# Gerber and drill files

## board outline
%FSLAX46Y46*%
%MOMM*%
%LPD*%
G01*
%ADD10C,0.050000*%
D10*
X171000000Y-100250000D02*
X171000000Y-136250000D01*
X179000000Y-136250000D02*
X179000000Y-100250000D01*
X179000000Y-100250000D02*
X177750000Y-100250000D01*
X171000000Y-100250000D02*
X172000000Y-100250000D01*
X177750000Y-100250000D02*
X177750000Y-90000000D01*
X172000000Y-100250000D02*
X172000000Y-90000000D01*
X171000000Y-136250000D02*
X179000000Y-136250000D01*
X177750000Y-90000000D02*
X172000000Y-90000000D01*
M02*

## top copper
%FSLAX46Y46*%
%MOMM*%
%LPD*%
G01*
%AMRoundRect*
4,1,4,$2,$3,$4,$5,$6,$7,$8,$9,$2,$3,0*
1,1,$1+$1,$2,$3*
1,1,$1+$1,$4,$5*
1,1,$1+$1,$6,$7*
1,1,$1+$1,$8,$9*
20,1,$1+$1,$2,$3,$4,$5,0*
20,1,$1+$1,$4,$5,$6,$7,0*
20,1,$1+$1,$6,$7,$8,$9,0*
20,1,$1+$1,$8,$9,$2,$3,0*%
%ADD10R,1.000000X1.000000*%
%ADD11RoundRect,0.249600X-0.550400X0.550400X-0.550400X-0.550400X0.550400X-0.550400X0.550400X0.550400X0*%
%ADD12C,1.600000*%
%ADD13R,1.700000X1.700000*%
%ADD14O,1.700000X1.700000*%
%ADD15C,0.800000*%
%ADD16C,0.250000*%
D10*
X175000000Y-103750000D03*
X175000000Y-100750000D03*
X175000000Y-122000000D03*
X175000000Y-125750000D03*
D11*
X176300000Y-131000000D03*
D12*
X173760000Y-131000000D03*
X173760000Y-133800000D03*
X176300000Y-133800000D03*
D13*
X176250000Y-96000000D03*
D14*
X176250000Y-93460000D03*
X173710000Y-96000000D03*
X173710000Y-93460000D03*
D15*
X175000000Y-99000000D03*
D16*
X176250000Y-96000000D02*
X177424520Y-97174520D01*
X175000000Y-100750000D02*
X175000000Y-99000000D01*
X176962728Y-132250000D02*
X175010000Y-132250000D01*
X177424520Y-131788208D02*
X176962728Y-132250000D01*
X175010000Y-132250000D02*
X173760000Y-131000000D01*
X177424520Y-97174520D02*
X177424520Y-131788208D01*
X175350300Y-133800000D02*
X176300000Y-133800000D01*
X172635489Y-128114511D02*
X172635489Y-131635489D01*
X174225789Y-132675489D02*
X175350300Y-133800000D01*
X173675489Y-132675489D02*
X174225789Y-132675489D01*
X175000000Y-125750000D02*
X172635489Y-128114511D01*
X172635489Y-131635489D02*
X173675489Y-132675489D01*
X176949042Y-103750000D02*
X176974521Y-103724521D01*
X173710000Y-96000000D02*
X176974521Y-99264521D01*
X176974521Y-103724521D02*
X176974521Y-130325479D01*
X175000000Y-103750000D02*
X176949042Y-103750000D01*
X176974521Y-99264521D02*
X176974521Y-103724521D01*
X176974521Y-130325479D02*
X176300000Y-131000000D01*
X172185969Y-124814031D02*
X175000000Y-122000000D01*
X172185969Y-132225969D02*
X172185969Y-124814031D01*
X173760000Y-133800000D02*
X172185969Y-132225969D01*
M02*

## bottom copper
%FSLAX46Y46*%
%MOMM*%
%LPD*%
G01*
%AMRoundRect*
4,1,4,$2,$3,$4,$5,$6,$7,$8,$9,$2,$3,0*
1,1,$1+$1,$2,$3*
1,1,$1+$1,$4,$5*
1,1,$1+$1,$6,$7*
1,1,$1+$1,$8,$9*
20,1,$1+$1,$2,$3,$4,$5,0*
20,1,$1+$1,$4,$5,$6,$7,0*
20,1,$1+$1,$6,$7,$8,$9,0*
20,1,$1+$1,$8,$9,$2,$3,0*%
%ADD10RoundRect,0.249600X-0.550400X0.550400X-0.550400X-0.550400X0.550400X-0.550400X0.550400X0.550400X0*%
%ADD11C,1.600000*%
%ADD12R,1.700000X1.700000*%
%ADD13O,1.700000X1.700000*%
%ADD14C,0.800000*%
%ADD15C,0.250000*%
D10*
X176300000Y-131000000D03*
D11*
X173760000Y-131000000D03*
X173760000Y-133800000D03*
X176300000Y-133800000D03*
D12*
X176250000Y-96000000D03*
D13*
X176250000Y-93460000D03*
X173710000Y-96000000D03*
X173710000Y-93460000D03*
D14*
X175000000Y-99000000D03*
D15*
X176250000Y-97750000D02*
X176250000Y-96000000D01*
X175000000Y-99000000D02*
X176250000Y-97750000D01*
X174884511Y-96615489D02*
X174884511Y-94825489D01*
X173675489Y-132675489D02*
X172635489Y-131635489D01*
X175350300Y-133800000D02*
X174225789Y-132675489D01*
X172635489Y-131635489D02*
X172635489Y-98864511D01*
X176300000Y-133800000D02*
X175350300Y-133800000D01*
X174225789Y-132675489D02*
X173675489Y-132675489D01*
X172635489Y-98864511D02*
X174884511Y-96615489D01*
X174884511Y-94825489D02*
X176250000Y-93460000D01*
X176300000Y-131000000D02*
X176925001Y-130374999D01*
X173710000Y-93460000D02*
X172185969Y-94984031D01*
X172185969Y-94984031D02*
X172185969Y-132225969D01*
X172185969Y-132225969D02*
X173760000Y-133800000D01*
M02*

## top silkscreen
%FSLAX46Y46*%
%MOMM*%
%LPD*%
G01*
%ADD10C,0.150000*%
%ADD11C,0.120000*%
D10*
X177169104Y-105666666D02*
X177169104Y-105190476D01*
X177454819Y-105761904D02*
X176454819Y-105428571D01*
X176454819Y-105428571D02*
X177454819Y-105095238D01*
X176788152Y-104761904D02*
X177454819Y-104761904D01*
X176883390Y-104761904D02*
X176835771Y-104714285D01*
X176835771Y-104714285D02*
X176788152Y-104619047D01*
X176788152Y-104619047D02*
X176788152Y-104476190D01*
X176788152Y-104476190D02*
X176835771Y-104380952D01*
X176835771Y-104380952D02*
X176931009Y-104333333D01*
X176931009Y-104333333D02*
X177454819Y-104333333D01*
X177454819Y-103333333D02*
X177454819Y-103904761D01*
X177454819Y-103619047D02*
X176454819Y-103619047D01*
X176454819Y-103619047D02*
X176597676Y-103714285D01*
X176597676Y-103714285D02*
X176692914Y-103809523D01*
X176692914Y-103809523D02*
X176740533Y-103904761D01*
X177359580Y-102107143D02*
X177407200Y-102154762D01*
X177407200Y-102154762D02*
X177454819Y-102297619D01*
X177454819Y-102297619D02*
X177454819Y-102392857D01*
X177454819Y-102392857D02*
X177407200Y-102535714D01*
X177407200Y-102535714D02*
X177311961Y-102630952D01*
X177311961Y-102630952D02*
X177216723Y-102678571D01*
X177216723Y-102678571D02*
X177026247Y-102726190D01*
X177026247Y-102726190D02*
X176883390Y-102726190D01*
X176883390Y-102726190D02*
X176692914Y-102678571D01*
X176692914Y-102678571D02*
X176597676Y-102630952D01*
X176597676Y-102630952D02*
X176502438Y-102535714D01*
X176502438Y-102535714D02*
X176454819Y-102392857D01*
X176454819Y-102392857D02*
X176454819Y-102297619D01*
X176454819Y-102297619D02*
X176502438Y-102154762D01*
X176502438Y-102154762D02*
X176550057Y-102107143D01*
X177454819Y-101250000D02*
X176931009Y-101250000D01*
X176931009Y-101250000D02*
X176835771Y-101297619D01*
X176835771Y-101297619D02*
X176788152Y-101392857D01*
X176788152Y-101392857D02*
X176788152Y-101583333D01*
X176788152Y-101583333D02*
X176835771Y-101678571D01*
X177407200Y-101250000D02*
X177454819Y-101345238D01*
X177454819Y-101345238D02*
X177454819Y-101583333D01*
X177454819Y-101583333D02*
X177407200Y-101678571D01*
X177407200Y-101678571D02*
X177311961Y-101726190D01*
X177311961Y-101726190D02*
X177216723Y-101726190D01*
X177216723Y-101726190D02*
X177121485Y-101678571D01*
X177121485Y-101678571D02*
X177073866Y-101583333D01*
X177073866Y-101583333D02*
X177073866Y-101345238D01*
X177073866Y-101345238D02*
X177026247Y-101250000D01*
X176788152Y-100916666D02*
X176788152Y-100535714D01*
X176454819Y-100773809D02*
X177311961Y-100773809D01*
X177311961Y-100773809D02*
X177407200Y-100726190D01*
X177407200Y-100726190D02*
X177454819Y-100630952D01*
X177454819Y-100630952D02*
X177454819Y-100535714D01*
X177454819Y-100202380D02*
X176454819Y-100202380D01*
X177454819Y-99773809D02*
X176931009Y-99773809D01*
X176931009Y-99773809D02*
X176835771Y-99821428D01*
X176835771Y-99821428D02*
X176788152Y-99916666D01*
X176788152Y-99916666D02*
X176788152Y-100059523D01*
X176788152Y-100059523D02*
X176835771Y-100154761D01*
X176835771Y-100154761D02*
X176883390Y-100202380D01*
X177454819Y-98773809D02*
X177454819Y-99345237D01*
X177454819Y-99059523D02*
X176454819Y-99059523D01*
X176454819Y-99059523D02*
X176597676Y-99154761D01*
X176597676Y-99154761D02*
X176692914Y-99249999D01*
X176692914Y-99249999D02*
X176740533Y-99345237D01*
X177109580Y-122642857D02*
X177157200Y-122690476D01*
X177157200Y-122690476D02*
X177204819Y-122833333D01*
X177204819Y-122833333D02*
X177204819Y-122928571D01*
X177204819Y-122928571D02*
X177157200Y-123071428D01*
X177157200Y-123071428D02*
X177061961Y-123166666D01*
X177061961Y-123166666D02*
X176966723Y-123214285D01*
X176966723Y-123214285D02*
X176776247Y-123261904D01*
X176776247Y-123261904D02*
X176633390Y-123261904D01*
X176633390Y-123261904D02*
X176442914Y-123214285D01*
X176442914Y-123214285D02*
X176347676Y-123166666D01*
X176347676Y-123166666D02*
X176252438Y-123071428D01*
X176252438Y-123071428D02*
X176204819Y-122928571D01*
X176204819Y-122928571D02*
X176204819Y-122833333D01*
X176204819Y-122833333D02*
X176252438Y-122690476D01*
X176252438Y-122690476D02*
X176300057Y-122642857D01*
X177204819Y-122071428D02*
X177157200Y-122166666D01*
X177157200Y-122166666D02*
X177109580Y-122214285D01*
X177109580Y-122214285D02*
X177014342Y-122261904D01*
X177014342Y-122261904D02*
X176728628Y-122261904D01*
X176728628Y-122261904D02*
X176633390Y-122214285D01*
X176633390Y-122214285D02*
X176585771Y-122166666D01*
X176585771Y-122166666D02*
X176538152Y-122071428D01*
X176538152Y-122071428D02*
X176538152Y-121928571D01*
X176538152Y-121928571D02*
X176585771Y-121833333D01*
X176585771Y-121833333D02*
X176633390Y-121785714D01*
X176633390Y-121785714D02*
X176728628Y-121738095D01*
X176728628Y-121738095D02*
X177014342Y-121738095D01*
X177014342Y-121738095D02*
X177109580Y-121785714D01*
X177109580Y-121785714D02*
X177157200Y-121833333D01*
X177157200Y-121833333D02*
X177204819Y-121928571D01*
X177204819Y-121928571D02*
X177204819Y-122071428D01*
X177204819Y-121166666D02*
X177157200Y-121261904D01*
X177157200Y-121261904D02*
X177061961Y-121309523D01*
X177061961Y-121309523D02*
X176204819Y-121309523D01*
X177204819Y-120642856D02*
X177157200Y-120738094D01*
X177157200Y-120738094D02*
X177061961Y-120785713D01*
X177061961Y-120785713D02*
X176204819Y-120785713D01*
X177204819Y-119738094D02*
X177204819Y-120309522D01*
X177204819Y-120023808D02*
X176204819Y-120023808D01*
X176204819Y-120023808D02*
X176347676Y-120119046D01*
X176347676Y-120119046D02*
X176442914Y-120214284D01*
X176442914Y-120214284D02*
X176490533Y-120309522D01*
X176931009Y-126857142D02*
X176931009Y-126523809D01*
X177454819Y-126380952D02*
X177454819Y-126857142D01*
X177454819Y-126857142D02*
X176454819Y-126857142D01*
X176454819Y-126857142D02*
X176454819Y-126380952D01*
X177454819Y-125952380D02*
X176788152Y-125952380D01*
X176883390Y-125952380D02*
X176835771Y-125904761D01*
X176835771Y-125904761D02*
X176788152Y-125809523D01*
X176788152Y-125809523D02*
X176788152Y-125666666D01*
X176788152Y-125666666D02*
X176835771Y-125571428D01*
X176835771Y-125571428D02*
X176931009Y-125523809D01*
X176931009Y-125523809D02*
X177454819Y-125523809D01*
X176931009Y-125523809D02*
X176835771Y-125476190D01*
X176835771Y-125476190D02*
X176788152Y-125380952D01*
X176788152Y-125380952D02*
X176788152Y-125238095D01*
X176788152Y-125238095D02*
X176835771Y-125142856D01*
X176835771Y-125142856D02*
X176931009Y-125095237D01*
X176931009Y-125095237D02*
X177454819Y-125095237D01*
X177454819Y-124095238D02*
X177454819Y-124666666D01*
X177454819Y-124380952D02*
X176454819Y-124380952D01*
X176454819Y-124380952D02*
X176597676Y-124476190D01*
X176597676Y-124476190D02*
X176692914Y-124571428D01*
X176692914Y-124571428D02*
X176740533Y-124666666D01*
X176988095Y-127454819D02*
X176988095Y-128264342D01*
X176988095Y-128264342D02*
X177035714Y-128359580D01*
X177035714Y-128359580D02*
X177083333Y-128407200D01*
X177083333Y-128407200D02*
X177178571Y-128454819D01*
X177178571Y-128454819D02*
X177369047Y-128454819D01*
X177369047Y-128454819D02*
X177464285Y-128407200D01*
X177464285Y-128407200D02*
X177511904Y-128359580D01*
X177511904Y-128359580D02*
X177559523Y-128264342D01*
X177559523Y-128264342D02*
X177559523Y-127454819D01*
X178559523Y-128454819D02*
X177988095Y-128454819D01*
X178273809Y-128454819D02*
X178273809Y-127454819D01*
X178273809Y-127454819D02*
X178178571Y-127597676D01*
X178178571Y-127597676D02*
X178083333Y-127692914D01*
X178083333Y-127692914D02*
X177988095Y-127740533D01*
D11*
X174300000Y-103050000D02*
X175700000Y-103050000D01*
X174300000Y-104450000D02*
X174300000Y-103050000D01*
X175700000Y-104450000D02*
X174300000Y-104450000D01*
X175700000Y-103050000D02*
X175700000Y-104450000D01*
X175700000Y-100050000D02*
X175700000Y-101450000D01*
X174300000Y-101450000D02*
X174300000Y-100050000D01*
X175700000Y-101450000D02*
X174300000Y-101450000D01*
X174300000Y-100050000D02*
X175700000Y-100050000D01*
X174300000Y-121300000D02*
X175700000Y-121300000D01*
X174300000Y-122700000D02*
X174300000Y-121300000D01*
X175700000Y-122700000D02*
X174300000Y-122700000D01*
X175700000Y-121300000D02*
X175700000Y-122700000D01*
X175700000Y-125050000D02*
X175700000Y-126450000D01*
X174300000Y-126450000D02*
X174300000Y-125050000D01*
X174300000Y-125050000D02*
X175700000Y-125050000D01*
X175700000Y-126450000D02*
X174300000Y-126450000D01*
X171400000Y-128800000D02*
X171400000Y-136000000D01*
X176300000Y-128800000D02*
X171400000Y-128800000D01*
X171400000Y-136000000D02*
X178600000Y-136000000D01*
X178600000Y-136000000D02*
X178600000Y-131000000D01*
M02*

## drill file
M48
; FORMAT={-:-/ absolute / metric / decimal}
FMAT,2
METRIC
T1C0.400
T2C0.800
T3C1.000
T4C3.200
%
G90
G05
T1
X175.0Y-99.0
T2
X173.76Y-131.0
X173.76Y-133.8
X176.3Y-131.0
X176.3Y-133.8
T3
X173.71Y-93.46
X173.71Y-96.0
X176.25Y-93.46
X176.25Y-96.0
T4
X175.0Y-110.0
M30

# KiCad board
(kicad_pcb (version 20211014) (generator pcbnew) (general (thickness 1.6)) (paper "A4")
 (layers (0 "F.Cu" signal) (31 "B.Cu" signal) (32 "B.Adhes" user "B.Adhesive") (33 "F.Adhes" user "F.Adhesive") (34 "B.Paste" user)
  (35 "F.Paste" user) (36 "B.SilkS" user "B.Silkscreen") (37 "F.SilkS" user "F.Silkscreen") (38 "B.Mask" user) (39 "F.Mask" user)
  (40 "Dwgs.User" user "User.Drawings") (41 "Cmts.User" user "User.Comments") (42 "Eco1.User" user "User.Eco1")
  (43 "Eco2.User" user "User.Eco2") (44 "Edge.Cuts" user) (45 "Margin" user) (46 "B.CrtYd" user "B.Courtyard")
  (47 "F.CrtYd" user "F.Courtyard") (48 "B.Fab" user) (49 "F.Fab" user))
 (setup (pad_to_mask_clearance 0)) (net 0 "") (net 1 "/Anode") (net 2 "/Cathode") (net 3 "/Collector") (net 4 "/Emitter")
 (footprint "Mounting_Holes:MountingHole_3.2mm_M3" (layer "F.Cu") (at 175 110)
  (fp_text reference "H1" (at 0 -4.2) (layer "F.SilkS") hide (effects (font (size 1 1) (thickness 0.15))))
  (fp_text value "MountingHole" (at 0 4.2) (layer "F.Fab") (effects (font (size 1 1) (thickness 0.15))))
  (pad "" np_thru_hole circle locked (at 0 0) (size 3.2 3.2) (drill 3.2) (layers *.Cu *.Mask)))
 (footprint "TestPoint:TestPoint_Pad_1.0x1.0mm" (layer "F.Cu") (at 175 103.75)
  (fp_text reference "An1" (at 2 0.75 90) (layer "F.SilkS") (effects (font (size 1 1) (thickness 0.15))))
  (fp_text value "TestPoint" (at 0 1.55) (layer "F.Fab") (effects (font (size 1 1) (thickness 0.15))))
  (fp_line (start -0.7 -0.7) (end 0.7 -0.7) (layer "F.SilkS") (width 0.12))
  (fp_line (start -0.7 0.7) (end -0.7 -0.7) (layer "F.SilkS") (width 0.12))
  (fp_line (start 0.7 0.7) (end -0.7 0.7) (layer "F.SilkS") (width 0.12))
  (fp_line (start 0.7 -0.7) (end 0.7 0.7) (layer "F.SilkS") (width 0.12))
  (pad "1" smd rect locked (at 0 0) (size 1 1) (layers "F.Cu" "F.Mask") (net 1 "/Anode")))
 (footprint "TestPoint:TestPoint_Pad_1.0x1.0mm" (layer "F.Cu") (at 175 100.75)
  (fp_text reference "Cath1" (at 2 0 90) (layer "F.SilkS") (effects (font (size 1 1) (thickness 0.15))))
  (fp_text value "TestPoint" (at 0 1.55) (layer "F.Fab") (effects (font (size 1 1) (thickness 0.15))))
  (fp_line (start 0.7 -0.7) (end 0.7 0.7) (layer "F.SilkS") (width 0.12))
  (fp_line (start -0.7 0.7) (end -0.7 -0.7) (layer "F.SilkS") (width 0.12))
  (fp_line (start 0.7 0.7) (end -0.7 0.7) (layer "F.SilkS") (width 0.12))
  (fp_line (start -0.7 -0.7) (end 0.7 -0.7) (layer "F.SilkS") (width 0.12))
  (pad "1" smd rect locked (at 0 0) (size 1 1) (layers "F.Cu" "F.Mask") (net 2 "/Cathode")))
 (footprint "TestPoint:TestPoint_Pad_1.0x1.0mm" (layer "F.Cu") (at 175 122)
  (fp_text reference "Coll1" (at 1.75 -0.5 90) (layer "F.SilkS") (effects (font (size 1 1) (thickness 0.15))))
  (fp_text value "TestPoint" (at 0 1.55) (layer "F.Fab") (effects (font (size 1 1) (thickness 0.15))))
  (fp_line (start -0.7 -0.7) (end 0.7 -0.7) (layer "F.SilkS") (width 0.12))
  (fp_line (start -0.7 0.7) (end -0.7 -0.7) (layer "F.SilkS") (width 0.12))
  (fp_line (start 0.7 0.7) (end -0.7 0.7) (layer "F.SilkS") (width 0.12))
  (fp_line (start 0.7 -0.7) (end 0.7 0.7) (layer "F.SilkS") (width 0.12))
  (pad "1" smd rect locked (at 0 0) (size 1 1) (layers "F.Cu" "F.Mask") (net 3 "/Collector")))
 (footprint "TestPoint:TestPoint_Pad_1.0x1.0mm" (layer "F.Cu") (at 175 125.75)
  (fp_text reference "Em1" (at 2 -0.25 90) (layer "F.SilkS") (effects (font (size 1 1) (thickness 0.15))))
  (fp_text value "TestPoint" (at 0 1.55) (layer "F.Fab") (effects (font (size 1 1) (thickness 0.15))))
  (fp_line (start 0.7 -0.7) (end 0.7 0.7) (layer "F.SilkS") (width 0.12))
  (fp_line (start -0.7 0.7) (end -0.7 -0.7) (layer "F.SilkS") (width 0.12))
  (fp_line (start -0.7 -0.7) (end 0.7 -0.7) (layer "F.SilkS") (width 0.12))
  (fp_line (start 0.7 0.7) (end -0.7 0.7) (layer "F.SilkS") (width 0.12))
  (pad "1" smd rect locked (at 0 0) (size 1 1) (layers "F.Cu" "F.Mask") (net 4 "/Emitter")))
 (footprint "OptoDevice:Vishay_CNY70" (layer "F.Cu") (at 176.3 131 -90)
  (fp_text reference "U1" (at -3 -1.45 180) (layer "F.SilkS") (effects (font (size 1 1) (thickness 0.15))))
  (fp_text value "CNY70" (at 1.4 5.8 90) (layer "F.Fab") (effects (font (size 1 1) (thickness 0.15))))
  (fp_line (start -2.2 4.9) (end 5 4.9) (layer "F.SilkS") (width 0.12))
  (fp_line (start -2.2 0) (end -2.2 4.9) (layer "F.SilkS") (width 0.12))
  (fp_line (start 5 4.9) (end 5 -2.3) (layer "F.SilkS") (width 0.12))
  (fp_line (start 5 -2.3) (end 0 -2.3) (layer "F.SilkS") (width 0.12))
  (pad "1" thru_hole roundrect locked (at 0 0 270) (size 1.6 1.6) (drill 0.8) (layers *.Cu *.Mask) (roundrect_rratio 0.156) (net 1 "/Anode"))
  (pad "2" thru_hole circle locked (at 0 2.54 270) (size 1.6 1.6) (drill 0.8) (layers *.Cu *.Mask) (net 2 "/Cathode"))
  (pad "3" thru_hole circle locked (at 2.8 2.54 270) (size 1.6 1.6) (drill 0.8) (layers *.Cu *.Mask) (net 3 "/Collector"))
  (pad "4" thru_hole circle locked (at 2.8 0 270) (size 1.6 1.6) (drill 0.8) (layers *.Cu *.Mask) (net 4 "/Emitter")))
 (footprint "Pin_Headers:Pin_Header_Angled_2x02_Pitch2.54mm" (layer "B.Cu") (at 176.25 96 90)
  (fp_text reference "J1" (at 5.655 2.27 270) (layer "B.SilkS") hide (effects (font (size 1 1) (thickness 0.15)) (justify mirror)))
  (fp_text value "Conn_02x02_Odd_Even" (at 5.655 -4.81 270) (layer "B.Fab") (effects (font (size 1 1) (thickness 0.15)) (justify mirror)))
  (pad "1" thru_hole rect (at 0 0 90) (size 1.7 1.7) (drill 1) (layers *.Cu *.Mask) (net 2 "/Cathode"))
  (pad "2" thru_hole oval (at 2.54 0 90) (size 1.7 1.7) (drill 1) (layers *.Cu *.Mask) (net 4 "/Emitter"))
  (pad "3" thru_hole oval (at 0 -2.54 90) (size 1.7 1.7) (drill 1) (layers *.Cu *.Mask) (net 1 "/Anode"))
  (pad "4" thru_hole oval (at 2.54 -2.54 90) (size 1.7 1.7) (drill 1) (layers *.Cu *.Mask) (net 3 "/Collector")))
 (gr_line (start 171 100.25) (end 171 136.25) (layer "Edge.Cuts") (width 0.05))
 (gr_line (start 179 136.25) (end 179 100.25) (layer "Edge.Cuts") (width 0.05))
 (gr_line (start 179 100.25) (end 177.75 100.25) (layer "Edge.Cuts") (width 0.05))
 (gr_line (start 171 100.25) (end 172 100.25) (layer "Edge.Cuts") (width 0.05))
 (gr_line (start 177.75 100.25) (end 177.75 90) (layer "Edge.Cuts") (width 0.05))
 (gr_line (start 172 100.25) (end 172 90) (layer "Edge.Cuts") (width 0.05))
 (gr_line (start 171 136.25) (end 179 136.25) (layer "Edge.Cuts") (width 0.05))
 (gr_line (start 177.75 90) (end 172 90) (layer "Edge.Cuts") (width 0.05))
 (segment (start 176.25 96) (end 177.42452 97.17452) (width 0.25) (layer "F.Cu") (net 2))
 (segment (start 175 100.75) (end 175 99) (width 0.25) (layer "F.Cu") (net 2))
 (segment (start 176.962728 132.25) (end 175.01 132.25) (width 0.25) (layer "F.Cu") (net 2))
 (segment (start 177.42452 131.788208) (end 176.962728 132.25) (width 0.25) (layer "F.Cu") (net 2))
 (segment (start 175.01 132.25) (end 173.76 131) (width 0.25) (layer "F.Cu") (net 2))
 (segment (start 177.42452 97.17452) (end 177.42452 131.788208) (width 0.25) (layer "F.Cu") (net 2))
 (via (at 175 99) (size 0.8) (drill 0.4) (layers "F.Cu" "B.Cu") (free) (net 2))
 (segment (start 176.25 97.75) (end 176.25 96) (width 0.25) (layer "B.Cu") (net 2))
 (segment (start 175 99) (end 176.25 97.75) (width 0.25) (layer "B.Cu") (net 2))
 (segment (start 175.3503 133.8) (end 176.3 133.8) (width 0.25) (layer "F.Cu") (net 4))
 (segment (start 172.635489 128.114511) (end 172.635489 131.635489) (width 0.25) (layer "F.Cu") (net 4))
 (segment (start 174.225789 132.675489) (end 175.3503 133.8) (width 0.25) (layer "F.Cu") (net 4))
 (segment (start 173.675489 132.675489) (end 174.225789 132.675489) (width 0.25) (layer "F.Cu") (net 4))
 (segment (start 175 125.75) (end 172.635489 128.114511) (width 0.25) (layer "F.Cu") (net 4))
 (segment (start 172.635489 131.635489) (end 173.675489 132.675489) (width 0.25) (layer "F.Cu") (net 4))
 (segment (start 174.884511 96.615489) (end 174.884511 94.825489) (width 0.25) (layer "B.Cu") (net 4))
 (segment (start 173.675489 132.675489) (end 172.635489 131.635489) (width 0.25) (layer "B.Cu") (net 4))
 (segment (start 175.3503 133.8) (end 174.225789 132.675489) (width 0.25) (layer "B.Cu") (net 4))
 (segment (start 172.635489 131.635489) (end 172.635489 98.864511) (width 0.25) (layer "B.Cu") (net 4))
 (segment (start 176.3 133.8) (end 175.3503 133.8) (width 0.25) (layer "B.Cu") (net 4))
 (segment (start 174.225789 132.675489) (end 173.675489 132.675489) (width 0.25) (layer "B.Cu") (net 4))
 (segment (start 172.635489 98.864511) (end 174.884511 96.615489) (width 0.25) (layer "B.Cu") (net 4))
 (segment (start 174.884511 94.825489) (end 176.25 93.46) (width 0.25) (layer "B.Cu") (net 4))
 (segment (start 176.949042 103.75) (end 176.974521 103.724521) (width 0.25) (layer "F.Cu") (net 1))
 (segment (start 173.71 96) (end 176.974521 99.264521) (width 0.25) (layer "F.Cu") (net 1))
 (segment (start 176.974521 103.724521) (end 176.974521 130.325479) (width 0.25) (layer "F.Cu") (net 1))
 (segment (start 175 103.75) (end 176.949042 103.75) (width 0.25) (layer "F.Cu") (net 1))
 (segment (start 176.974521 99.264521) (end 176.974521 103.724521) (width 0.25) (layer "F.Cu") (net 1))
 (segment (start 176.974521 130.325479) (end 176.3 131) (width 0.25) (layer "F.Cu") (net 1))
 (segment (start 176.3 131) (end 176.925001 130.374999) (width 0.25) (layer "B.Cu") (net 1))
 (segment (start 172.185969 124.814031) (end 175 122) (width 0.25) (layer "F.Cu") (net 3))
 (segment (start 172.185969 132.225969) (end 172.185969 124.814031) (width 0.25) (layer "F.Cu") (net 3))
 (segment (start 173.76 133.8) (end 172.185969 132.225969) (width 0.25) (layer "F.Cu") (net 3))
 (segment (start 173.71 93.46) (end 172.185969 94.984031) (width 0.25) (layer "B.Cu") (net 3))
 (segment (start 172.185969 94.984031) (end 172.185969 132.225969) (width 0.25) (layer "B.Cu") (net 3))
 (segment (start 172.185969 132.225969) (end 173.76 133.8) (width 0.25) (layer "B.Cu") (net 3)))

